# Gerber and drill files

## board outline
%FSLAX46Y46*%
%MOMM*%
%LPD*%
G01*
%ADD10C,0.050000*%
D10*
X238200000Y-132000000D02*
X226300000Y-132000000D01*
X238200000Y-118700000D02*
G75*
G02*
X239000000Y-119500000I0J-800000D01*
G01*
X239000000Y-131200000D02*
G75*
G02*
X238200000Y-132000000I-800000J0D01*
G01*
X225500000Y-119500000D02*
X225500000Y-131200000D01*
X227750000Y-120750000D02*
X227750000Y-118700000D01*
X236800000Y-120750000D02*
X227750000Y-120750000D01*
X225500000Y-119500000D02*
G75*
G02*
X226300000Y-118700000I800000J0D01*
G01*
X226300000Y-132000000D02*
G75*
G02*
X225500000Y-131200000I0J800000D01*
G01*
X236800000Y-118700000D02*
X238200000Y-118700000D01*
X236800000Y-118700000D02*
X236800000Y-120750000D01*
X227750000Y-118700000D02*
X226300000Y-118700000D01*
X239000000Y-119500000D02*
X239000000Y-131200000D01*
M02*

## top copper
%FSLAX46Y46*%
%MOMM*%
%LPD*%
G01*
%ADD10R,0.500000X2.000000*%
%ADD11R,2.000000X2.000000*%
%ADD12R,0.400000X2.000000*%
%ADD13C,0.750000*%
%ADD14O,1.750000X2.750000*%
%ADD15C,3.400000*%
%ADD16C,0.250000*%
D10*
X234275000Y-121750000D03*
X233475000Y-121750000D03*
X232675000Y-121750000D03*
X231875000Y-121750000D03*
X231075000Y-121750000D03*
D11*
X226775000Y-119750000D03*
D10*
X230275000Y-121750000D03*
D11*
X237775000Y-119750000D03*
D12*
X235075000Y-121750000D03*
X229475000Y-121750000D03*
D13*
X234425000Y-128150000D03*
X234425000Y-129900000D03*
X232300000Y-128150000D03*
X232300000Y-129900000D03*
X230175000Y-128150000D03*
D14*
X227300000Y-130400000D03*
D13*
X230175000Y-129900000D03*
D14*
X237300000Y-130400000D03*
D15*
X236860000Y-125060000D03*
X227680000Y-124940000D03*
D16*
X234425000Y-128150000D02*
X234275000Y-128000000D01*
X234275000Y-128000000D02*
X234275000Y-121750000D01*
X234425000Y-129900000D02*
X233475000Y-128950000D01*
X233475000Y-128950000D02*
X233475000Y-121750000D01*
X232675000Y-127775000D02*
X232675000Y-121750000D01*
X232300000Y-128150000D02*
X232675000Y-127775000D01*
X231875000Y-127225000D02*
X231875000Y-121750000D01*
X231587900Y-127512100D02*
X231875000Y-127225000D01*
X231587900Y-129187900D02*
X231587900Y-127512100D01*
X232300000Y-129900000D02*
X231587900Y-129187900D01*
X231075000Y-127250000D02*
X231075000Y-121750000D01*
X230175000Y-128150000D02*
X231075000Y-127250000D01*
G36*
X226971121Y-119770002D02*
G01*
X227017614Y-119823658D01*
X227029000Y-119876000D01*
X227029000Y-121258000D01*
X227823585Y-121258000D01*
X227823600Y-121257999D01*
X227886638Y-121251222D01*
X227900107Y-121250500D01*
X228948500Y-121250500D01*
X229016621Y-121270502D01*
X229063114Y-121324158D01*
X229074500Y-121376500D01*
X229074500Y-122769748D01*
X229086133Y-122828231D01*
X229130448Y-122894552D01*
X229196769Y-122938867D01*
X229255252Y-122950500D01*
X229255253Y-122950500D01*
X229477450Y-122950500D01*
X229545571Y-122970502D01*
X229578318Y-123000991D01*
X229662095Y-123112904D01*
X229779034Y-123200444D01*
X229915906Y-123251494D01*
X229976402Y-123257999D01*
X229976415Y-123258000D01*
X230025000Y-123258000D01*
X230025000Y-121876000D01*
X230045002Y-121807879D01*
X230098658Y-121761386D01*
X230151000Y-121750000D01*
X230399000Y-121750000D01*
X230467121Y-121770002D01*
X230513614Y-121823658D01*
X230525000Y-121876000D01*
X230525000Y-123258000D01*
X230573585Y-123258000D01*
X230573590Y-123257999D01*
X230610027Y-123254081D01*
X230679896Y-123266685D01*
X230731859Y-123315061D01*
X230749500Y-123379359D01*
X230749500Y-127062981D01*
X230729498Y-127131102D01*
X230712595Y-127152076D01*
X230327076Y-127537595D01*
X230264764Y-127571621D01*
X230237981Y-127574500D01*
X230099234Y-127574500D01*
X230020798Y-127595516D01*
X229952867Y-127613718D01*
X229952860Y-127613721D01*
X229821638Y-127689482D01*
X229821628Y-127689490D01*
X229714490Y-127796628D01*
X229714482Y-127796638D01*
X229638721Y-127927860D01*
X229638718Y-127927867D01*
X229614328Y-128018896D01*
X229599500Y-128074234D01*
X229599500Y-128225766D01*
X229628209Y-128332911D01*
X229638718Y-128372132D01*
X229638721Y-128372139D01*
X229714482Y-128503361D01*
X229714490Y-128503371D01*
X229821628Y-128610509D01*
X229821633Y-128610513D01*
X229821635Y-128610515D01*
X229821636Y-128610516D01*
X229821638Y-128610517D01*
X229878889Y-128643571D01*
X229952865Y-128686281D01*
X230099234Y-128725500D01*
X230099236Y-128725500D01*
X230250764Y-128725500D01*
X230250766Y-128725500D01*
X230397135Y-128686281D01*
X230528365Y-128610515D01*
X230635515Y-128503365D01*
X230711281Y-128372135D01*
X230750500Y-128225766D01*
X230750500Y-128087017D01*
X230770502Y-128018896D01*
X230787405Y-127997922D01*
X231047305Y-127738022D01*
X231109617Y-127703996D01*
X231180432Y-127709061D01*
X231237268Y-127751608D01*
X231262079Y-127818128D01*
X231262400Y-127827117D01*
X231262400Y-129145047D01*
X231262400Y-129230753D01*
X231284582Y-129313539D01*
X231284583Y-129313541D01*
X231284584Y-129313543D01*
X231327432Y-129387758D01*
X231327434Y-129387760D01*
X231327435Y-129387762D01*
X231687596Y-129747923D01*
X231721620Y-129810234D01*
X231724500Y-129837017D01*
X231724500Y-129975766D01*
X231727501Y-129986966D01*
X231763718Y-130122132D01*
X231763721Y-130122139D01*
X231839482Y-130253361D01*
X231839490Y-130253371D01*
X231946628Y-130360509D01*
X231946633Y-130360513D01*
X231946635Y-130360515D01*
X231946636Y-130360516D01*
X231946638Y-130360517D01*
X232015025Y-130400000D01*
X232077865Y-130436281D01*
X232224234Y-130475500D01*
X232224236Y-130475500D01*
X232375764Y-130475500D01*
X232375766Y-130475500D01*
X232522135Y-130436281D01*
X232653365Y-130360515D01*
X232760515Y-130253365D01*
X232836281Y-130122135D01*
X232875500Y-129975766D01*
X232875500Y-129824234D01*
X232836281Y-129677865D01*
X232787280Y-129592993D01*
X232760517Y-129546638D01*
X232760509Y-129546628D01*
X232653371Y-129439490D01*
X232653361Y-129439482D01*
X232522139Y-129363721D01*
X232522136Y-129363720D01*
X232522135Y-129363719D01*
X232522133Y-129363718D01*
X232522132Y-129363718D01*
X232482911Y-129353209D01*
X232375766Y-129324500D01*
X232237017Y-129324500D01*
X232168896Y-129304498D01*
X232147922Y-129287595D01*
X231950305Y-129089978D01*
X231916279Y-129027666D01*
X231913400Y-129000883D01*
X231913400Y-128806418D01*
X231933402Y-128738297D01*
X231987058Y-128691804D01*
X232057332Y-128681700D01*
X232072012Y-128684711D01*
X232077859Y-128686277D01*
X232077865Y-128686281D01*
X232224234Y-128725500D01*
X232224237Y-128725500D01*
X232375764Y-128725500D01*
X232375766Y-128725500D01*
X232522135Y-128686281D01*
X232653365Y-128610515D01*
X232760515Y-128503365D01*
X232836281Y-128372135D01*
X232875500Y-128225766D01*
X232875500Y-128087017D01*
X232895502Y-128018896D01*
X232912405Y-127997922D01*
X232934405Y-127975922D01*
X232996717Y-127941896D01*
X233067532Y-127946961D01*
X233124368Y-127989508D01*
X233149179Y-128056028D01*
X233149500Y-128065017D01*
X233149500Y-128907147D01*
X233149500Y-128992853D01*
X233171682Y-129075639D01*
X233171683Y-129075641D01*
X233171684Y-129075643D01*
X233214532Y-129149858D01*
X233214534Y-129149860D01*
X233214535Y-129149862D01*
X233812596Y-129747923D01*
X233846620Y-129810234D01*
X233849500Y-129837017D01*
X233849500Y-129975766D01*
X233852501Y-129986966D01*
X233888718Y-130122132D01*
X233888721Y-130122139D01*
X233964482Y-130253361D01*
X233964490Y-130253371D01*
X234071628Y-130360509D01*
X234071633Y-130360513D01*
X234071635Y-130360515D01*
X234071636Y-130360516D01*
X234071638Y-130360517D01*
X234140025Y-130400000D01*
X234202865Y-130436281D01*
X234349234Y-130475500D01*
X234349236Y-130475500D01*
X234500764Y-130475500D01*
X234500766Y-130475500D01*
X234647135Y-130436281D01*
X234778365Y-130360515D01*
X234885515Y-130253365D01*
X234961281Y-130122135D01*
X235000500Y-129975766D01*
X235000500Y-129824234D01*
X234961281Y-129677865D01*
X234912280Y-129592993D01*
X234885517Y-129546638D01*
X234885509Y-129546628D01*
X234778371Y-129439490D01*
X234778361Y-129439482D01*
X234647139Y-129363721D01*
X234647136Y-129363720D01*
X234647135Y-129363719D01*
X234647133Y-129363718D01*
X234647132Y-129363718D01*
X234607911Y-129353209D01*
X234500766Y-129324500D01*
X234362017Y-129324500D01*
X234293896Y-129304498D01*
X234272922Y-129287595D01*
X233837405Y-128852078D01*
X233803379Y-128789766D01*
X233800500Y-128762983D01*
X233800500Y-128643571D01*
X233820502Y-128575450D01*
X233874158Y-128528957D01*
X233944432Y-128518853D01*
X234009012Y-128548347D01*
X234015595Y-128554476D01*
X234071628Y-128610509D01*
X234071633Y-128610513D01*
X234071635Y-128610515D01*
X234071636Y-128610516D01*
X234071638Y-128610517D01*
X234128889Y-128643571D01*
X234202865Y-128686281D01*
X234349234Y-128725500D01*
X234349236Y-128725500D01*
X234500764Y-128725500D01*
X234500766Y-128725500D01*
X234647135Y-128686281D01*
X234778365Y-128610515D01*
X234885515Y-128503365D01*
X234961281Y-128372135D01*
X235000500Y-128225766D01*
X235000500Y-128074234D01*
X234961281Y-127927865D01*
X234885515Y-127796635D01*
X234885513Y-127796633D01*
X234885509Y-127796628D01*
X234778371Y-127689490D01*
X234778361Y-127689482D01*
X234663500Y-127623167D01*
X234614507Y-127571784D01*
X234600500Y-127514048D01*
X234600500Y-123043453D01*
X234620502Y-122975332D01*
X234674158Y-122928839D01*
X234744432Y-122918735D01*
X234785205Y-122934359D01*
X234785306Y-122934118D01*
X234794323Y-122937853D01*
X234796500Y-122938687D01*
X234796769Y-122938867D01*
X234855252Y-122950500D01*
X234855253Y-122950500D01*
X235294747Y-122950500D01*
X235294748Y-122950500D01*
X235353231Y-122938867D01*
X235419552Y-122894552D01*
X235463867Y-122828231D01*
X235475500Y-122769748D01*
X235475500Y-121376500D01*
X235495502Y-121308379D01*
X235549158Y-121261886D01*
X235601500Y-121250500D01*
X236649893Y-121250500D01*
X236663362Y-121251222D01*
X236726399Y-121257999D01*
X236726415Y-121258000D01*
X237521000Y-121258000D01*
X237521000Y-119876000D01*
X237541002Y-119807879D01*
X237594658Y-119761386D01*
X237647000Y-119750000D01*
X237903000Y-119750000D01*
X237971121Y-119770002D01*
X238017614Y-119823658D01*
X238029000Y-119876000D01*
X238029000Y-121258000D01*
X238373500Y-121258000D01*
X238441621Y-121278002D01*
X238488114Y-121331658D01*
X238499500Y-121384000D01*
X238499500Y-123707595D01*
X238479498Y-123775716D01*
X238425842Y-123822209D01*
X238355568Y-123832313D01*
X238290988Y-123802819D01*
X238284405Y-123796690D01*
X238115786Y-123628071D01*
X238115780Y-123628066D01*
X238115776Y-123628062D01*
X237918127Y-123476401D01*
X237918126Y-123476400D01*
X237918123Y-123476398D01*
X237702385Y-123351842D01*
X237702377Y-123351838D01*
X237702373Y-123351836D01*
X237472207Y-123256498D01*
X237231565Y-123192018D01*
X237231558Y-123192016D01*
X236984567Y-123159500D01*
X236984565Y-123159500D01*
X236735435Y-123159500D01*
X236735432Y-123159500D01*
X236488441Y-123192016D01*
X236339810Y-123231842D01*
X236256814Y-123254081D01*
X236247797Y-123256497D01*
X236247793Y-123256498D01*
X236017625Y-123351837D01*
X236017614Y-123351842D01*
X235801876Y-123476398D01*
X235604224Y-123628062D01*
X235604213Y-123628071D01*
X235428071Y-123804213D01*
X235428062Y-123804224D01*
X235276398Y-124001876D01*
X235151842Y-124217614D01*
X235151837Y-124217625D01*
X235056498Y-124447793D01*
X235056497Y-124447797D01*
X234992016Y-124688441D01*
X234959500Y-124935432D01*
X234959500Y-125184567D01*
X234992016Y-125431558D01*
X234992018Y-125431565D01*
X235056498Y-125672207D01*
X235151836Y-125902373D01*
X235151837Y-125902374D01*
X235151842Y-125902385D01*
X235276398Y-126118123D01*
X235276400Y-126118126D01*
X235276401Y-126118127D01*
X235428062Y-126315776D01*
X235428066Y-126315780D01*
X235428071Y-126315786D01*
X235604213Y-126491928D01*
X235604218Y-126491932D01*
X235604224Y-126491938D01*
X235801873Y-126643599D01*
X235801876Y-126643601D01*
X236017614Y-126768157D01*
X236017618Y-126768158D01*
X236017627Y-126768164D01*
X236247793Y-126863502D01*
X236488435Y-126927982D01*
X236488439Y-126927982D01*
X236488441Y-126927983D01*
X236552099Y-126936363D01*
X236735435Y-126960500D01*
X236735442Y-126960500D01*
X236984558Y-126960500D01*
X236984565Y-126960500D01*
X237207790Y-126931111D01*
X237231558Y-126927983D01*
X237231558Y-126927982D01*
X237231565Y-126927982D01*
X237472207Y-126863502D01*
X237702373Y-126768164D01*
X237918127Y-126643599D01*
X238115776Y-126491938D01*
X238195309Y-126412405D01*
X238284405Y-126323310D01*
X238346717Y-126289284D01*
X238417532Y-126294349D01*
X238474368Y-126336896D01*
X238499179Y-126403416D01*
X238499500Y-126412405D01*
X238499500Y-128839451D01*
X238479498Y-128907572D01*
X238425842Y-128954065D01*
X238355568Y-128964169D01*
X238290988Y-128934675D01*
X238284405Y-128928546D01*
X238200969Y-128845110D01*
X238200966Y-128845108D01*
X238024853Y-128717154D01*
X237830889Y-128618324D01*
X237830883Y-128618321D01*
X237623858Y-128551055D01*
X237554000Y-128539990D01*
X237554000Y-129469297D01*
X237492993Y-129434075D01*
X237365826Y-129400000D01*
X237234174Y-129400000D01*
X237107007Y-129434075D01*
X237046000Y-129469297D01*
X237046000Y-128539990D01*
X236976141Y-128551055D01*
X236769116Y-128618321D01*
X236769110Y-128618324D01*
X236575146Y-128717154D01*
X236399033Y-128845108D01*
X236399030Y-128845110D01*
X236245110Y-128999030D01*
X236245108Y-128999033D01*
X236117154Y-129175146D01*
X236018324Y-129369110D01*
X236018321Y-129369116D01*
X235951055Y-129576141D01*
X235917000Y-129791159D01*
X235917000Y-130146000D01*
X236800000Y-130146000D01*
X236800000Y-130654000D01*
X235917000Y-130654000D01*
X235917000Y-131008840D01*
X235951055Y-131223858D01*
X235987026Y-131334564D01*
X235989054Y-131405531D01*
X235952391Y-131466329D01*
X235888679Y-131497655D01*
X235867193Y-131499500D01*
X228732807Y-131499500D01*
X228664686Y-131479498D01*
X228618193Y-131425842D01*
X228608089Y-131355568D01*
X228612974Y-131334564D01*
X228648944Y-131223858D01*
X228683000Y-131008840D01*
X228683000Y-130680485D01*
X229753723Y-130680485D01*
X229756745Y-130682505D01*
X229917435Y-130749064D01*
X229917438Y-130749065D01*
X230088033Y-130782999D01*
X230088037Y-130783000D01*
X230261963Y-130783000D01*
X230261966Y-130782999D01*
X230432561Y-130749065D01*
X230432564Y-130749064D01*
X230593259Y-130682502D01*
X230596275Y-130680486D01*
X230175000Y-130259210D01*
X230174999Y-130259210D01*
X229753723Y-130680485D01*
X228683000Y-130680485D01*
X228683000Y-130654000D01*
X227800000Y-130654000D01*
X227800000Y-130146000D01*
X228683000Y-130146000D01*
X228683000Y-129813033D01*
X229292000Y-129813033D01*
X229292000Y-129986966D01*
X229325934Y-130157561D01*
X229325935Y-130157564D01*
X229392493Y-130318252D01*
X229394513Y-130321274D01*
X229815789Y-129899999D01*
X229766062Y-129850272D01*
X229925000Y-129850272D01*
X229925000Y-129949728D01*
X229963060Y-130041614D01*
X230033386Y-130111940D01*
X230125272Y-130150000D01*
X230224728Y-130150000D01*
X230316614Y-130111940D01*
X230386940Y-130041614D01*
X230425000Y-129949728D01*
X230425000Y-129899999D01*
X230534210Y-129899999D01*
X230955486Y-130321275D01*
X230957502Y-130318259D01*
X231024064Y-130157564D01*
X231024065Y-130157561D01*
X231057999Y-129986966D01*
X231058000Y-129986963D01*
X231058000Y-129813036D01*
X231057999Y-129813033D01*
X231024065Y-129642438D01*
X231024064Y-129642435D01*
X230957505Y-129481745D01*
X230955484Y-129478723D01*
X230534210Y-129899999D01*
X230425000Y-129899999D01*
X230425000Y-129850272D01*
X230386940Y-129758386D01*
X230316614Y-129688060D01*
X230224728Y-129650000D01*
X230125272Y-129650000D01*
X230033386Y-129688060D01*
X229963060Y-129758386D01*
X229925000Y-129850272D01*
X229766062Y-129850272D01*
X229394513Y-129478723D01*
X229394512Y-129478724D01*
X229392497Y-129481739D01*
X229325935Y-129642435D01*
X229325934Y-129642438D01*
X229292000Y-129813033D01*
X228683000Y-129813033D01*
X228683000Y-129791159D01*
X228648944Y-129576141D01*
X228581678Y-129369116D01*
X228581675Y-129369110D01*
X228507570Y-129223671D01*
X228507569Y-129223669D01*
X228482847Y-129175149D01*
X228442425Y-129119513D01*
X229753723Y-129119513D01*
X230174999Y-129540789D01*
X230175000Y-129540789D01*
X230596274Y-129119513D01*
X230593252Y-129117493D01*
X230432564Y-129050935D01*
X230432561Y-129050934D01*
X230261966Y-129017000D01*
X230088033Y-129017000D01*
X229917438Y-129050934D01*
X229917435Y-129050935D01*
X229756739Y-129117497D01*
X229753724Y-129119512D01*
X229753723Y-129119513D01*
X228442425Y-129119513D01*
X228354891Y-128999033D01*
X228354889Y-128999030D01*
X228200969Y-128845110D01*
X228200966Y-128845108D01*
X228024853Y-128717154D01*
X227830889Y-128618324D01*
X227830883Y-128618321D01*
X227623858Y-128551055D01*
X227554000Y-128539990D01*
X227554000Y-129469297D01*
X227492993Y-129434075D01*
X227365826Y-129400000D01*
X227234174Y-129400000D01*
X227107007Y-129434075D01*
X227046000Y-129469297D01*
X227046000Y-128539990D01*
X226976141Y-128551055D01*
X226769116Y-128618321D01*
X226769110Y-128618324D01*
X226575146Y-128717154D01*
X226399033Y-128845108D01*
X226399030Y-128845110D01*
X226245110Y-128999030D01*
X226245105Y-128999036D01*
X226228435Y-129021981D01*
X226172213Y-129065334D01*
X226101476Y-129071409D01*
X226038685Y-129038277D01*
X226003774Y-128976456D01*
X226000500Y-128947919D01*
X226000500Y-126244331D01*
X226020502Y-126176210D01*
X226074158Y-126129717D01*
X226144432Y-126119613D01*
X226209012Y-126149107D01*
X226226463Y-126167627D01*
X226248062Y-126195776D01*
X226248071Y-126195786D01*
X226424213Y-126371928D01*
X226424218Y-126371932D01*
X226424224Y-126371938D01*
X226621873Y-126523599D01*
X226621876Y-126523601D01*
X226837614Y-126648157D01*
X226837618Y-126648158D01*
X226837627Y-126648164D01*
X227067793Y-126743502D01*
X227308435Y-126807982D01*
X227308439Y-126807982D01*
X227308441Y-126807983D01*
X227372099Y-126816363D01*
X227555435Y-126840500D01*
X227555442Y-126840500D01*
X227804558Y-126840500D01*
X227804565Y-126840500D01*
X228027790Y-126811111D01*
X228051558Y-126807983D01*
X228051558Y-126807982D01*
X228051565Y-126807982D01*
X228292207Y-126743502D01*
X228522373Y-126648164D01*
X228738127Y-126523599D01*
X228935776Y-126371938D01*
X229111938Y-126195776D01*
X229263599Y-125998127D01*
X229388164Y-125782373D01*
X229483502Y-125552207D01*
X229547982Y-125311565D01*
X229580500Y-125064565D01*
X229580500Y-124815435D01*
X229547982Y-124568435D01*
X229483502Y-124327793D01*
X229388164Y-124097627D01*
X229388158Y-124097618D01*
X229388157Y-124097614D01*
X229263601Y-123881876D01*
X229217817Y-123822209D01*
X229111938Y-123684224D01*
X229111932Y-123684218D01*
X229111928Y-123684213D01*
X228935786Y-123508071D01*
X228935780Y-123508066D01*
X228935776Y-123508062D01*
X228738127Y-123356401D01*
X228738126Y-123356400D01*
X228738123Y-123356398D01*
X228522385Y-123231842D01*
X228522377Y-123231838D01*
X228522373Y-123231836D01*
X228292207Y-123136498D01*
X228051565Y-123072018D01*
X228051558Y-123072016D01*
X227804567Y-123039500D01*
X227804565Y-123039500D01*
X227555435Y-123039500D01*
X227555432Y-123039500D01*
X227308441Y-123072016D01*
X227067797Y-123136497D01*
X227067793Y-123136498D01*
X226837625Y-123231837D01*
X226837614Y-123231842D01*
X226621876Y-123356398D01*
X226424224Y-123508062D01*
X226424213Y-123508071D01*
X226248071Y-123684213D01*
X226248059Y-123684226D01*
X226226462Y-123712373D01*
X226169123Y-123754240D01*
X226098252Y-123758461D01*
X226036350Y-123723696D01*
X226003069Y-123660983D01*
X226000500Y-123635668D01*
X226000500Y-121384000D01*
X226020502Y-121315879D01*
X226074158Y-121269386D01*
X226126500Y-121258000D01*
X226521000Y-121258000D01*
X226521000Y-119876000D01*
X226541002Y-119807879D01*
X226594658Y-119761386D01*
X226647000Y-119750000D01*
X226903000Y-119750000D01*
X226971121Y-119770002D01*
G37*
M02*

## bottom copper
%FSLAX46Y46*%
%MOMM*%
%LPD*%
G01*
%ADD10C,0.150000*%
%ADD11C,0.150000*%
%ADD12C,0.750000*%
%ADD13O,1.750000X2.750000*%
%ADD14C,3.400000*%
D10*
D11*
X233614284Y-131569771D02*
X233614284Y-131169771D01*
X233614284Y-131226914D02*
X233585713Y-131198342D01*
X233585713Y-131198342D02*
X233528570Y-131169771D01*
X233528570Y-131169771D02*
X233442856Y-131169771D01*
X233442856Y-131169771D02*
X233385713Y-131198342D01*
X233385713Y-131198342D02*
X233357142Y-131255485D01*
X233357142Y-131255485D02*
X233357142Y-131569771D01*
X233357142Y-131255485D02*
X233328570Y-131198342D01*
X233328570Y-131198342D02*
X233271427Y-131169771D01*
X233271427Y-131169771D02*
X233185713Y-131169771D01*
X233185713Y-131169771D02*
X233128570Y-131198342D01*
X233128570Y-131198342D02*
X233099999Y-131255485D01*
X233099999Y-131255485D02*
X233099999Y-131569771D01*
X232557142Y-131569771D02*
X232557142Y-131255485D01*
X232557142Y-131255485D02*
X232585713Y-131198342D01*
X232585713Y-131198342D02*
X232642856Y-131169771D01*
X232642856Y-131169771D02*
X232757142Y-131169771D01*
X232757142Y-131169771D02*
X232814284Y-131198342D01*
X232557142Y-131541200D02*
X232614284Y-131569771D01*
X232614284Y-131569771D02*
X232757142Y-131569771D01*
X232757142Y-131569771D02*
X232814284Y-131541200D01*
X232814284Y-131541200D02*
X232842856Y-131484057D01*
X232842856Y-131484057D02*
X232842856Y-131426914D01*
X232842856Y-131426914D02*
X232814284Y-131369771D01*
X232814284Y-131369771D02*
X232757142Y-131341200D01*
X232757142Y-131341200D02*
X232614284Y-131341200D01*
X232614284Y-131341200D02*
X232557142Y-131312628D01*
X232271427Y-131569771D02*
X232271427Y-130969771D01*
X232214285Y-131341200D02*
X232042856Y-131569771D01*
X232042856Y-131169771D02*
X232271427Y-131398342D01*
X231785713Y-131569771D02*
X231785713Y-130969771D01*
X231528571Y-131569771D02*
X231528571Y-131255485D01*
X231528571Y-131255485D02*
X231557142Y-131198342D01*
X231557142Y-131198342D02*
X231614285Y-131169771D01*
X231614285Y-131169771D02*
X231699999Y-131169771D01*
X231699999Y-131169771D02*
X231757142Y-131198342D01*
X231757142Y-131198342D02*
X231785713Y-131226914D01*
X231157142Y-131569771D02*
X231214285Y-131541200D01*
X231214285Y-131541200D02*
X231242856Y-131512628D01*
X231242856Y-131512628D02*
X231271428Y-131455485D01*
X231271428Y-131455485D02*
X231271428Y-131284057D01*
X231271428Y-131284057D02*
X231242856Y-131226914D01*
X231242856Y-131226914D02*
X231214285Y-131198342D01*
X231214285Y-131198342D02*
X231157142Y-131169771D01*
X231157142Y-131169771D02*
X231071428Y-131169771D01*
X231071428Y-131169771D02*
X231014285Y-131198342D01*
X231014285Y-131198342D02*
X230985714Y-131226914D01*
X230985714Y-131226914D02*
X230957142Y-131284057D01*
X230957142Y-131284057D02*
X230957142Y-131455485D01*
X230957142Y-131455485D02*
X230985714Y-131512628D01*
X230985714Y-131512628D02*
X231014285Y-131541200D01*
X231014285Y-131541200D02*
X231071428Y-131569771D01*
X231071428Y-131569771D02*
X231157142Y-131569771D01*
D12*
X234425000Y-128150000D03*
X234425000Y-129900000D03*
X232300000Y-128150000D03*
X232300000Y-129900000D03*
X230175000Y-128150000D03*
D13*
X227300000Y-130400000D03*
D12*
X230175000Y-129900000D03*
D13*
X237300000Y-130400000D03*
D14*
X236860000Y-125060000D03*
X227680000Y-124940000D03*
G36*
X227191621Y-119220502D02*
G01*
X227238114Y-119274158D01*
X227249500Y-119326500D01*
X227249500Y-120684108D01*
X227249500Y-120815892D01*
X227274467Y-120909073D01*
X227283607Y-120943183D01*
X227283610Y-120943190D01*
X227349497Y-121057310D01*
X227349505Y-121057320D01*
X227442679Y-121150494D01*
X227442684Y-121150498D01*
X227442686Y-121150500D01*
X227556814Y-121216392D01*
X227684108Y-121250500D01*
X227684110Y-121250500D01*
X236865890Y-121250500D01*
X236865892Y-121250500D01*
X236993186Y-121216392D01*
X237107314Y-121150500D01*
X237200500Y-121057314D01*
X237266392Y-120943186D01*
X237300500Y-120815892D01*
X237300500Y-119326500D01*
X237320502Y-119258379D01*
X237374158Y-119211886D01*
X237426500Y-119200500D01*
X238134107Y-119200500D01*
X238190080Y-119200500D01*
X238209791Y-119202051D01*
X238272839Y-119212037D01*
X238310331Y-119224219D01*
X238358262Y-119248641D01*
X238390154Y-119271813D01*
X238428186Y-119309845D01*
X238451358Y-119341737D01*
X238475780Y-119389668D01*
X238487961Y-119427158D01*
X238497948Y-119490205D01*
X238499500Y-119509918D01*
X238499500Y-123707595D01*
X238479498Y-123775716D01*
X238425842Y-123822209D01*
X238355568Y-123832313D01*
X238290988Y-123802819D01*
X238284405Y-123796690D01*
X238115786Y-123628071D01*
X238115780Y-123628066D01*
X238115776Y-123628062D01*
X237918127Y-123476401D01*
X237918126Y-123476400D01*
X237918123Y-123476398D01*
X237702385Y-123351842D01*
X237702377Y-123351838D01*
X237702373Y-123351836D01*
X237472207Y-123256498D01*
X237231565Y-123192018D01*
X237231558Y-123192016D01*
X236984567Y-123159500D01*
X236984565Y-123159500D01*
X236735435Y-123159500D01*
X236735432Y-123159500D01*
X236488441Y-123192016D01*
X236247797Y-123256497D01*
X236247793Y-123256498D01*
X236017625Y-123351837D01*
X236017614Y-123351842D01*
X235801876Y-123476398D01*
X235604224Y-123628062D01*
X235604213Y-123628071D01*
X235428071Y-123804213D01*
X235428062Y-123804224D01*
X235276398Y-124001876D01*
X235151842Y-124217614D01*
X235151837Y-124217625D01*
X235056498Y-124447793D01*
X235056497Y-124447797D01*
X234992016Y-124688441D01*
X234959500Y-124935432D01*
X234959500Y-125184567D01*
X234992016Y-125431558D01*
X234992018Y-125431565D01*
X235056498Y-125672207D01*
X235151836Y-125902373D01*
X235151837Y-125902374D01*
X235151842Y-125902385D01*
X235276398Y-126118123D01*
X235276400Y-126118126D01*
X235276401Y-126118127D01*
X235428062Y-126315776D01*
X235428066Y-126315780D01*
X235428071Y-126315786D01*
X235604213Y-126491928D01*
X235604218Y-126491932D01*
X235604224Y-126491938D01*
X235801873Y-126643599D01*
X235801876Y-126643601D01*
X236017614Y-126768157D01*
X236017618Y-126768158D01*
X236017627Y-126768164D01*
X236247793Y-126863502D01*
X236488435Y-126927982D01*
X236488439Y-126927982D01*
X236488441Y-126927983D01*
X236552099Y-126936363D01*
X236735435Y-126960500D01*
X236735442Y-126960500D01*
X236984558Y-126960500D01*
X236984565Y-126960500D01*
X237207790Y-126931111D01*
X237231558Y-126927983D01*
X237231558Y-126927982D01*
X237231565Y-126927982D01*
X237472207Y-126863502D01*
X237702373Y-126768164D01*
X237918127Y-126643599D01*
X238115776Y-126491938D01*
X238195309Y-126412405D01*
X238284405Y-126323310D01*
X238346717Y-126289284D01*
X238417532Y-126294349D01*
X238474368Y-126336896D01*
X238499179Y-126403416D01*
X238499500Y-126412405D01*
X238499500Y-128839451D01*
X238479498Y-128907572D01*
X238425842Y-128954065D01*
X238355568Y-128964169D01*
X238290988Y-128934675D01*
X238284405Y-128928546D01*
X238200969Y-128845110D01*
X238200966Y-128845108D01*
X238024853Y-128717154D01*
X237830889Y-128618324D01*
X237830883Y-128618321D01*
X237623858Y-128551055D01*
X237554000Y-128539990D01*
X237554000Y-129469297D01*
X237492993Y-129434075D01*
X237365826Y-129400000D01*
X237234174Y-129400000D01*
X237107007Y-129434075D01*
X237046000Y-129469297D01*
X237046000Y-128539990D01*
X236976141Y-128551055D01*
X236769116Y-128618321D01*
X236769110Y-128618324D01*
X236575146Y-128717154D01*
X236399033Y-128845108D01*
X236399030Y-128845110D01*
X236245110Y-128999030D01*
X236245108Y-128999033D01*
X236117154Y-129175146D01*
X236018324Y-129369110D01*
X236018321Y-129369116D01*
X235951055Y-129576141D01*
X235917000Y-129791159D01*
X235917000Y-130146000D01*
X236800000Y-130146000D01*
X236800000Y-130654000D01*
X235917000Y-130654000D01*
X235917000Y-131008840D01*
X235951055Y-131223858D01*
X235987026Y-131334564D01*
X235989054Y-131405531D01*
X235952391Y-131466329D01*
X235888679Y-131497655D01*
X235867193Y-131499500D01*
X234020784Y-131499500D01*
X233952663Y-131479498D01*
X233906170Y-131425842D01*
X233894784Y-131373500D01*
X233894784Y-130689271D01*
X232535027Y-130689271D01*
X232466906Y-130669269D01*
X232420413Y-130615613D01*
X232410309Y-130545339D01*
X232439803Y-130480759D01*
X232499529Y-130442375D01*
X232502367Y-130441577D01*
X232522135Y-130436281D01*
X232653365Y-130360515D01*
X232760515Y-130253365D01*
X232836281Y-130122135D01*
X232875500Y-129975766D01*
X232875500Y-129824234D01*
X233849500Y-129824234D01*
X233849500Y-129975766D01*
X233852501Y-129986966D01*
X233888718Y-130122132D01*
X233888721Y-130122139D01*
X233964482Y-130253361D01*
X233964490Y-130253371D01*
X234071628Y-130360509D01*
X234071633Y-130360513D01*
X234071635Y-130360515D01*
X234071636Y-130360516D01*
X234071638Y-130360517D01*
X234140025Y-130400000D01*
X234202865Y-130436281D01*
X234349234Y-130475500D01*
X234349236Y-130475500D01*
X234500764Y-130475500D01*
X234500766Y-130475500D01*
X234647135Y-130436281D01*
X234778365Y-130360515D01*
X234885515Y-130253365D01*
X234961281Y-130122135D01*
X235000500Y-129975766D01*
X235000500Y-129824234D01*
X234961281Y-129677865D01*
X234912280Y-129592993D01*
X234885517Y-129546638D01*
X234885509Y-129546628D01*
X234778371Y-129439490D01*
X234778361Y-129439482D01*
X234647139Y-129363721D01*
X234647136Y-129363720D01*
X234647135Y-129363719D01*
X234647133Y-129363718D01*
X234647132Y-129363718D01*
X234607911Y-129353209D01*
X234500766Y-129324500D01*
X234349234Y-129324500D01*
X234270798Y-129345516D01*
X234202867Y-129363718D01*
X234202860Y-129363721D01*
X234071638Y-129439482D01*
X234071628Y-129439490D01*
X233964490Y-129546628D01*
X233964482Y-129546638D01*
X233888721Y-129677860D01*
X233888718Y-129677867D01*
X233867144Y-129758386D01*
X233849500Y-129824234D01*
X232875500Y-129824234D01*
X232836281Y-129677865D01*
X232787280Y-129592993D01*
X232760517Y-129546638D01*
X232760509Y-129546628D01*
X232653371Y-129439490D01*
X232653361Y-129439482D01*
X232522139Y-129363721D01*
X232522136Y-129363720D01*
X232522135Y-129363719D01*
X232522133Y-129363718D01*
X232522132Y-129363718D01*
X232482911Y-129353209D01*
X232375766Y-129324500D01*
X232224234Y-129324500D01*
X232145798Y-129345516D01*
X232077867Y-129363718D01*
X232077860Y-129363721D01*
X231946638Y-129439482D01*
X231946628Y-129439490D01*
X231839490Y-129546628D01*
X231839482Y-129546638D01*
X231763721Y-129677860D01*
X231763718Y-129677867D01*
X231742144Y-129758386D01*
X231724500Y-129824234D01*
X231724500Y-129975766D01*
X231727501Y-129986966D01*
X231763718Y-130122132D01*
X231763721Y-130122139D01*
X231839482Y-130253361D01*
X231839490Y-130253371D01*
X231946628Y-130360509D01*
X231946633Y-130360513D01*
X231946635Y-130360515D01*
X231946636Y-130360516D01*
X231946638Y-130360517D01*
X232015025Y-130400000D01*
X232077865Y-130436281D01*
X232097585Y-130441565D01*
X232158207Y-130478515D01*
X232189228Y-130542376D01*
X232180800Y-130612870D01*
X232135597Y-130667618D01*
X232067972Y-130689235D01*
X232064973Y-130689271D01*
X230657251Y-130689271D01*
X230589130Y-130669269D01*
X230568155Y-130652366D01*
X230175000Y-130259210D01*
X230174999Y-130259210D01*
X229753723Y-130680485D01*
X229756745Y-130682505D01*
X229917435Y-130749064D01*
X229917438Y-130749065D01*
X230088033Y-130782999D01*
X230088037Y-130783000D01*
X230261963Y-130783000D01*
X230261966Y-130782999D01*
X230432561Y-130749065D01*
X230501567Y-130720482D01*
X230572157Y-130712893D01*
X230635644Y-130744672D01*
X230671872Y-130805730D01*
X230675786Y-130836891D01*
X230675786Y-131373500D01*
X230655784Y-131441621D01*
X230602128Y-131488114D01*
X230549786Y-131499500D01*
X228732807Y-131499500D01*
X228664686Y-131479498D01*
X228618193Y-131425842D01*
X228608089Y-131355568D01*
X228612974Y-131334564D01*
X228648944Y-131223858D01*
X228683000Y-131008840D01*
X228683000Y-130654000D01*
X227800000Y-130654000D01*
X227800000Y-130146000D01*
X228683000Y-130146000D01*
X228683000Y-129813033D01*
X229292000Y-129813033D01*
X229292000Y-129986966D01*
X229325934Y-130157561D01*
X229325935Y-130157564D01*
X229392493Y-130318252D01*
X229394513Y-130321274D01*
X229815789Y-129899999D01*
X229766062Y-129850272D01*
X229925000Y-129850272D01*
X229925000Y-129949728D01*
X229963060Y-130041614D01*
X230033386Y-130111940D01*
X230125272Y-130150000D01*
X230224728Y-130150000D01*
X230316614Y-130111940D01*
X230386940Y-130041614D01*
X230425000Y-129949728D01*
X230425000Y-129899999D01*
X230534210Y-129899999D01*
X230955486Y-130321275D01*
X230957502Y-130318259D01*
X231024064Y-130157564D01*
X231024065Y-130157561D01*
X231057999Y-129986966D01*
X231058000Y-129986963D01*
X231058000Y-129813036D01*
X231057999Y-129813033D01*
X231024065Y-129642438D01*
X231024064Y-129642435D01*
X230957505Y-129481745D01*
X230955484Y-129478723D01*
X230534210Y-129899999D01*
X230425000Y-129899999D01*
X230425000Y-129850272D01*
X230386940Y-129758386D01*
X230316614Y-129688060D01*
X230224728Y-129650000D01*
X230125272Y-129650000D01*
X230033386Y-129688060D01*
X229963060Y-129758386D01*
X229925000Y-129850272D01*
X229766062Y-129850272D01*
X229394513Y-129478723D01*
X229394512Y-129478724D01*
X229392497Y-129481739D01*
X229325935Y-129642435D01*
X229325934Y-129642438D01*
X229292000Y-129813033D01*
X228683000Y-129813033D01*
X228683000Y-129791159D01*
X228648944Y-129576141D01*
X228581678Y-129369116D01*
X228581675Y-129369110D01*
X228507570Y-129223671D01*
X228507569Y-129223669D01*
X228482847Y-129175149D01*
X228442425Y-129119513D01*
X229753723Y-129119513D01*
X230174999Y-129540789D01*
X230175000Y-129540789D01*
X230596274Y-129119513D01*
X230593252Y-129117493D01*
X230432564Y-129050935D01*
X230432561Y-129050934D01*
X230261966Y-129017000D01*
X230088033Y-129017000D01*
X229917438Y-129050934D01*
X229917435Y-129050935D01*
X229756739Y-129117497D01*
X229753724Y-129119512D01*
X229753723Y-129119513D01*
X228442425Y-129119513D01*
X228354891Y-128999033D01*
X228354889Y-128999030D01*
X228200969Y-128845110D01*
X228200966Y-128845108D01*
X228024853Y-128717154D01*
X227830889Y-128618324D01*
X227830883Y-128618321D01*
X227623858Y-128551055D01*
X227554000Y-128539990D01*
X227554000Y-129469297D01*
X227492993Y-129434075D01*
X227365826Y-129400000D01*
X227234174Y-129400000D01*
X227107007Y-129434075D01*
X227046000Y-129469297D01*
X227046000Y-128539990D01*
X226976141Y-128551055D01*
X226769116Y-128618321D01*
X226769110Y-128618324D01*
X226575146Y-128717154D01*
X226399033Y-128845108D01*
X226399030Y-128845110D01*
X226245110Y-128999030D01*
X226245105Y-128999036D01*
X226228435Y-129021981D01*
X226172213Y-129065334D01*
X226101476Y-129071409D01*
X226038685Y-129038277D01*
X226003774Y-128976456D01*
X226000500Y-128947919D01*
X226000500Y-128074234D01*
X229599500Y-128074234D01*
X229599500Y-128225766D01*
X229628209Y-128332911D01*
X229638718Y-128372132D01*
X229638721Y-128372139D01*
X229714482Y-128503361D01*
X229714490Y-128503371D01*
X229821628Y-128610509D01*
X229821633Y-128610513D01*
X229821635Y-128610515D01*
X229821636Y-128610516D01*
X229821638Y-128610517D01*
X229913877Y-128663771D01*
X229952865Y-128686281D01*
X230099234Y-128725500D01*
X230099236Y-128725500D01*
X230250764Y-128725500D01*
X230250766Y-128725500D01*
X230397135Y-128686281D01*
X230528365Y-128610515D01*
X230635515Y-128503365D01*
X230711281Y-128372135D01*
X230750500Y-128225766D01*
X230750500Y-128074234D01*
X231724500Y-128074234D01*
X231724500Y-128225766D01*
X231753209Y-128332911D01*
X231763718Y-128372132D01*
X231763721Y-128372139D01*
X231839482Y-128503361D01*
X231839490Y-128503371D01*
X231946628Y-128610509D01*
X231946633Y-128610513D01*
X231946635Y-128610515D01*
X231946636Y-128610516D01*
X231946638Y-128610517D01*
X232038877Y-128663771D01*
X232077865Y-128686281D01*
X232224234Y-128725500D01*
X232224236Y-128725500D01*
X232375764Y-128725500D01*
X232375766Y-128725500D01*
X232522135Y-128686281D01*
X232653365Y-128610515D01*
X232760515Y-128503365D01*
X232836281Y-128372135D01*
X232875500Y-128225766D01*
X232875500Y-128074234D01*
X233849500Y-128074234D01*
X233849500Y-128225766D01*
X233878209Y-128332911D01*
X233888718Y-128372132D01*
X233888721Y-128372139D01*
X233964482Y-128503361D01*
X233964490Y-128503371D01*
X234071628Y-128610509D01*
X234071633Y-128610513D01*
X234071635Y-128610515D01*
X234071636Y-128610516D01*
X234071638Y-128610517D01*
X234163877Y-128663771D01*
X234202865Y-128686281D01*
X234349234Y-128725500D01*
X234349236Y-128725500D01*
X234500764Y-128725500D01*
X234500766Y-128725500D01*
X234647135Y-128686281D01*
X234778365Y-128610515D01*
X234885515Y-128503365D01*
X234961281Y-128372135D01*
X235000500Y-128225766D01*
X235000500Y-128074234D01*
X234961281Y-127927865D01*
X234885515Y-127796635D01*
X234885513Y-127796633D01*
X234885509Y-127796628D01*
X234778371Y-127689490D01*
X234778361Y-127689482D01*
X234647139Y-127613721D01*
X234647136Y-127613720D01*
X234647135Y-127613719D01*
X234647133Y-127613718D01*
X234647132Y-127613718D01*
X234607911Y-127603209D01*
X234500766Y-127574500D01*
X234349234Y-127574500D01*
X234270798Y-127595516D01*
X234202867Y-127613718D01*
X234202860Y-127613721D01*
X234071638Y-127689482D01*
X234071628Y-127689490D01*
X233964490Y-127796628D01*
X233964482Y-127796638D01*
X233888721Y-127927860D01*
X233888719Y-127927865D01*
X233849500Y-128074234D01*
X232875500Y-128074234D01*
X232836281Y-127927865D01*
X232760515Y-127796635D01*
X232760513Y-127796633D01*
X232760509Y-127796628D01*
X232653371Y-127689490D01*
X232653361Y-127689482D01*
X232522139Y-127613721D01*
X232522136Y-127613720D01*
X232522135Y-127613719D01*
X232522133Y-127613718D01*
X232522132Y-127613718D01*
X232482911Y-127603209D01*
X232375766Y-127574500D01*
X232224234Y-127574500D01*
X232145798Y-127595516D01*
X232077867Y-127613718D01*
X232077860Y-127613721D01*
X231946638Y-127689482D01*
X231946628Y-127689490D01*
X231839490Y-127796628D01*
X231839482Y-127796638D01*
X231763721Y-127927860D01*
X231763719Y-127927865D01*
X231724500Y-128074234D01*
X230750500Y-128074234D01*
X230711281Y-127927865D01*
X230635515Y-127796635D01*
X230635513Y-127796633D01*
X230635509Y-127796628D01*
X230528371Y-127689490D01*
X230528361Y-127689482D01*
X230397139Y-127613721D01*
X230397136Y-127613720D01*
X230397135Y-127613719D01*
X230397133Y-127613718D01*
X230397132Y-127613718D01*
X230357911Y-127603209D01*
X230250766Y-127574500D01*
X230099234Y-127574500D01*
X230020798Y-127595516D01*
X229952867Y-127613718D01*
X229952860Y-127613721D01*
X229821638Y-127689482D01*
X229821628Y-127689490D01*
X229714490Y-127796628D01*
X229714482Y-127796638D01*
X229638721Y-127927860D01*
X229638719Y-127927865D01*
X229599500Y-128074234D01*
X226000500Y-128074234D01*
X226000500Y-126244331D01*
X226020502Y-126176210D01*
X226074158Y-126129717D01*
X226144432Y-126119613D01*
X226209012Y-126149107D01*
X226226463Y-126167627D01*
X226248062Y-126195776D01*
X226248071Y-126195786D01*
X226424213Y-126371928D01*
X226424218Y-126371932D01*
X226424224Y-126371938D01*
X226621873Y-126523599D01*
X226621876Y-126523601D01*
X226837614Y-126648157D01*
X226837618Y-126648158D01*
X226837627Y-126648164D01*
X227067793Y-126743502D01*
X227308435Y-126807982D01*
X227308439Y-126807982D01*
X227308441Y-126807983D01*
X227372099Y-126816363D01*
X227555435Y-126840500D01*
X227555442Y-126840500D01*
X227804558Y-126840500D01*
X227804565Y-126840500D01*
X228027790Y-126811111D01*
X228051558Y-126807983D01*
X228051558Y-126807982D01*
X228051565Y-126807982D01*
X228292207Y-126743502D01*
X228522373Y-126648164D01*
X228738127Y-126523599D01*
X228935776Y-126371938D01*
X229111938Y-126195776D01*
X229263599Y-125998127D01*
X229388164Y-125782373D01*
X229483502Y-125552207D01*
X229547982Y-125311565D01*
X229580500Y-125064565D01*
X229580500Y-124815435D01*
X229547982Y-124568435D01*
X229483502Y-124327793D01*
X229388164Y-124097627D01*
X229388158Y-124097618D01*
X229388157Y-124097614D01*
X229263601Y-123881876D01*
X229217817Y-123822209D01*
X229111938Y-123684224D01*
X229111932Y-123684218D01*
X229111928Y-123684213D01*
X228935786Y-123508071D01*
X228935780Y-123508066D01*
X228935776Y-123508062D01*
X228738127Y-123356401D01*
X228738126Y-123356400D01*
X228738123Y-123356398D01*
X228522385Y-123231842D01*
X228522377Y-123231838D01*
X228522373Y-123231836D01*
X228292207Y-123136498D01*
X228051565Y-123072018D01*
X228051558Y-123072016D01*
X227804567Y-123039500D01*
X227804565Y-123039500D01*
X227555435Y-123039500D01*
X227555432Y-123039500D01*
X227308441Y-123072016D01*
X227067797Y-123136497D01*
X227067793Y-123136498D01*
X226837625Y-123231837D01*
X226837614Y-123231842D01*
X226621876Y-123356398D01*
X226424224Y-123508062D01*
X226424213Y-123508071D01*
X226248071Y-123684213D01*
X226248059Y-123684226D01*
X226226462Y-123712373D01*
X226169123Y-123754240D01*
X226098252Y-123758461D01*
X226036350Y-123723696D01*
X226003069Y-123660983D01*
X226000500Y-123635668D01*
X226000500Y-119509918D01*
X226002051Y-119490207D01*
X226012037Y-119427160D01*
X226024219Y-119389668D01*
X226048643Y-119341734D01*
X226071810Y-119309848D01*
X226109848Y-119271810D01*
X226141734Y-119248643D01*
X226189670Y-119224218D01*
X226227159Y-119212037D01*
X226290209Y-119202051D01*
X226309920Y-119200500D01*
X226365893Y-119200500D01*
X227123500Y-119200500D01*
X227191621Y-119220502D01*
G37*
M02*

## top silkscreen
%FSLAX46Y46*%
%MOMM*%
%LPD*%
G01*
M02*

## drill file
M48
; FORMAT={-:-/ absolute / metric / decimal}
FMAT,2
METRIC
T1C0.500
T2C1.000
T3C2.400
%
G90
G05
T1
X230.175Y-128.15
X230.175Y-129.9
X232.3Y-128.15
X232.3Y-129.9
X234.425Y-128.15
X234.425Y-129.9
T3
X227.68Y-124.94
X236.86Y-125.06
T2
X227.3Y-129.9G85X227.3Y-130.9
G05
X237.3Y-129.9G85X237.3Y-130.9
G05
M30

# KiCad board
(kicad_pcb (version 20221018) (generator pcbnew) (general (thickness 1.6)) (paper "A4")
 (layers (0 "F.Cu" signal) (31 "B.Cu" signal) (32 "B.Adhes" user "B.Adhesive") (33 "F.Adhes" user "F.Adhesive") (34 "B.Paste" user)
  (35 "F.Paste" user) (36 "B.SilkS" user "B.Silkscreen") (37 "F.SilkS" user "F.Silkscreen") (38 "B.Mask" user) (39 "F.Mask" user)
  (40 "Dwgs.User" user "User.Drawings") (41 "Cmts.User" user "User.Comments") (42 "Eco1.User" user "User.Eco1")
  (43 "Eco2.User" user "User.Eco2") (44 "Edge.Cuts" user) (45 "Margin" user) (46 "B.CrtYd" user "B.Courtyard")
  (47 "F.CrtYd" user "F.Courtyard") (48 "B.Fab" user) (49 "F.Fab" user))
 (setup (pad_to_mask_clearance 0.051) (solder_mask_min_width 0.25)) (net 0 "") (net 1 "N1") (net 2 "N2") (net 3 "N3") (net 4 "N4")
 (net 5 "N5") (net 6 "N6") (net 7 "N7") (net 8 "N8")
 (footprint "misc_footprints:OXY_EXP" (layer "F.Cu") (at 232.275 119.75)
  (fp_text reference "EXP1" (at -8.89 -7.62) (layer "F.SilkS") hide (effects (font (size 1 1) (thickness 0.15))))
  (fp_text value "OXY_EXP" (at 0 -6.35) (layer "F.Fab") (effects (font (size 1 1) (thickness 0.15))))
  (pad "1" smd rect (at 2 2) (size 0.5 2) (layers "F.Cu" "F.Paste" "F.Mask") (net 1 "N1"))
  (pad "2" smd rect (at 1.2 2) (size 0.5 2) (layers "F.Cu" "F.Paste" "F.Mask") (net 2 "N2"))
  (pad "3" smd rect (at 0.4 2) (size 0.5 2) (layers "F.Cu" "F.Paste" "F.Mask") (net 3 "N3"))
  (pad "4" smd rect (at -0.4 2) (size 0.5 2) (layers "F.Cu" "F.Paste" "F.Mask") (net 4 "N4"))
  (pad "5" smd rect (at -1.2 2) (size 0.5 2) (layers "F.Cu" "F.Paste" "F.Mask") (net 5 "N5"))
  (pad "6" smd rect (at -5.5 0) (size 2 2) (layers "F.Cu" "F.Paste" "F.Mask") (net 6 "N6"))
  (pad "6" smd rect (at -2 2) (size 0.5 2) (layers "F.Cu" "F.Paste" "F.Mask") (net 6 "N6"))
  (pad "6" smd rect (at 5.5 0) (size 2 2) (layers "F.Cu" "F.Paste" "F.Mask") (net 6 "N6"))
  (pad "7" smd rect (at 2.8 2) (size 0.4 2) (layers "F.Cu" "F.Paste" "F.Mask") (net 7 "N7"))
  (pad "8" smd rect (at -2.8 2) (size 0.4 2) (layers "F.Cu" "F.Paste" "F.Mask") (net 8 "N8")))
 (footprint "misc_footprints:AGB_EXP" (layer "F.Cu") (at 232.3 128.15)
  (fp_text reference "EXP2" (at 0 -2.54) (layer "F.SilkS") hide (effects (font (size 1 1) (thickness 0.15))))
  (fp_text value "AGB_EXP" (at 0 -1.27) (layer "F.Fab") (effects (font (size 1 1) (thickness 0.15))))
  (pad "1" thru_hole circle (at 2.125 0) (size 0.75 0.75) (drill 0.5) (layers "*.Cu" "*.Mask") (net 1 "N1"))
  (pad "2" thru_hole circle (at 2.125 1.75) (size 0.75 0.75) (drill 0.5) (layers "*.Cu" "*.Mask") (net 2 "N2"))
  (pad "3" thru_hole circle (at 0 0) (size 0.75 0.75) (drill 0.5) (layers "*.Cu" "*.Mask") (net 3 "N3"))
  (pad "4" thru_hole circle (at 0 1.75) (size 0.75 0.75) (drill 0.5) (layers "*.Cu" "*.Mask") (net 4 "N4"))
  (pad "5" thru_hole circle (at -2.125 0) (size 0.75 0.75) (drill 0.5) (layers "*.Cu" "*.Mask") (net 5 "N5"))
  (pad "6" thru_hole oval (at -5 2.25) (size 1.75 2.75) (drill oval 1 2) (layers "*.Cu" "*.Mask") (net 6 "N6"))
  (pad "6" thru_hole circle (at -2.125 1.75) (size 0.75 0.75) (drill 0.5) (layers "*.Cu" "*.Mask") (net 6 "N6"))
  (pad "6" thru_hole oval (at 5 2.25) (size 1.75 2.75) (drill oval 1 2) (layers "*.Cu" "*.Mask") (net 6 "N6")))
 (gr_line (start 238.2 132) (end 226.3 132) (stroke (width 0.05) (type solid)) (layer "Edge.Cuts"))
 (gr_arc (start 238.2 118.7) (mid 238.765685 118.934315) (end 239 119.5) (stroke (width 0.05) (type solid)) (layer "Edge.Cuts"))
 (gr_arc (start 239 131.2) (mid 238.765685 131.765685) (end 238.2 132) (stroke (width 0.05) (type solid)) (layer "Edge.Cuts"))
 (gr_line (start 225.5 119.5) (end 225.5 131.2) (stroke (width 0.05) (type solid)) (layer "Edge.Cuts"))
 (gr_line (start 227.75 120.75) (end 227.75 118.7) (stroke (width 0.05) (type solid)) (layer "Edge.Cuts"))
 (gr_line (start 236.8 120.75) (end 227.75 120.75) (stroke (width 0.05) (type solid)) (layer "Edge.Cuts"))
 (gr_arc (start 225.5 119.5) (mid 225.734315 118.934315) (end 226.3 118.7) (stroke (width 0.05) (type solid)) (layer "Edge.Cuts"))
 (gr_arc (start 226.3 132) (mid 225.734315 131.765685) (end 225.5 131.2) (stroke (width 0.05) (type solid)) (layer "Edge.Cuts"))
 (gr_line (start 236.8 118.7) (end 238.2 118.7) (stroke (width 0.05) (type solid)) (layer "Edge.Cuts"))
 (gr_line (start 236.8 118.7) (end 236.8 120.75) (stroke (width 0.05) (type solid)) (layer "Edge.Cuts"))
 (gr_line (start 227.75 118.7) (end 226.3 118.7) (stroke (width 0.05) (type solid)) (layer "Edge.Cuts"))
 (gr_line (start 239 119.5) (end 239 131.2) (stroke (width 0.05) (type solid)) (layer "Edge.Cuts"))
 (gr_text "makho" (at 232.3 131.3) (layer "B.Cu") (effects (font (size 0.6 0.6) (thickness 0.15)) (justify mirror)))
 (via (at 236.86 125.06) (size 3.4) (drill 2.4) (layers "F.Cu" "B.Cu") (free) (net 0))
 (via (at 227.68 124.94) (size 3.4) (drill 2.4) (layers "F.Cu" "B.Cu") (free) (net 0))
 (segment (start 234.425 128.15) (end 234.275 128) (width 0.25) (layer "F.Cu") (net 1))
 (segment (start 234.275 128) (end 234.275 121.75) (width 0.25) (layer "F.Cu") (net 1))
 (segment (start 234.425 129.9) (end 233.475 128.95) (width 0.25) (layer "F.Cu") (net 2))
 (segment (start 233.475 128.95) (end 233.475 121.75) (width 0.25) (layer "F.Cu") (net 2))
 (segment (start 232.675 127.775) (end 232.675 121.75) (width 0.25) (layer "F.Cu") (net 3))
 (segment (start 232.3 128.15) (end 232.675 127.775) (width 0.25) (layer "F.Cu") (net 3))
 (segment (start 231.875 127.225) (end 231.875 121.75) (width 0.25) (layer "F.Cu") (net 4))
 (segment (start 231.5879 127.5121) (end 231.875 127.225) (width 0.25) (layer "F.Cu") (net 4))
 (segment (start 231.5879 129.1879) (end 231.5879 127.5121) (width 0.25) (layer "F.Cu") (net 4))
 (segment (start 232.3 129.9) (end 231.5879 129.1879) (width 0.25) (layer "F.Cu") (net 4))
 (segment (start 231.075 127.25) (end 231.075 121.75) (width 0.25) (layer "F.Cu") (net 5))
 (segment (start 230.175 128.15) (end 231.075 127.25) (width 0.25) (layer "F.Cu") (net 5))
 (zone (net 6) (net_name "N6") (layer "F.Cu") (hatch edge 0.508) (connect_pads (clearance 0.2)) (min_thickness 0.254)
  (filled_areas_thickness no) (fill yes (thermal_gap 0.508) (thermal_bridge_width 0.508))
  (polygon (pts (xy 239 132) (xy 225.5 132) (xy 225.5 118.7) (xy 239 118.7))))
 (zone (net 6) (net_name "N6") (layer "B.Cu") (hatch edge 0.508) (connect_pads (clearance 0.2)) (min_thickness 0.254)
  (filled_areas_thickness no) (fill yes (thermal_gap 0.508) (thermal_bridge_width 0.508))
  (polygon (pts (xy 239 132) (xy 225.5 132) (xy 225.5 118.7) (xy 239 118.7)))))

